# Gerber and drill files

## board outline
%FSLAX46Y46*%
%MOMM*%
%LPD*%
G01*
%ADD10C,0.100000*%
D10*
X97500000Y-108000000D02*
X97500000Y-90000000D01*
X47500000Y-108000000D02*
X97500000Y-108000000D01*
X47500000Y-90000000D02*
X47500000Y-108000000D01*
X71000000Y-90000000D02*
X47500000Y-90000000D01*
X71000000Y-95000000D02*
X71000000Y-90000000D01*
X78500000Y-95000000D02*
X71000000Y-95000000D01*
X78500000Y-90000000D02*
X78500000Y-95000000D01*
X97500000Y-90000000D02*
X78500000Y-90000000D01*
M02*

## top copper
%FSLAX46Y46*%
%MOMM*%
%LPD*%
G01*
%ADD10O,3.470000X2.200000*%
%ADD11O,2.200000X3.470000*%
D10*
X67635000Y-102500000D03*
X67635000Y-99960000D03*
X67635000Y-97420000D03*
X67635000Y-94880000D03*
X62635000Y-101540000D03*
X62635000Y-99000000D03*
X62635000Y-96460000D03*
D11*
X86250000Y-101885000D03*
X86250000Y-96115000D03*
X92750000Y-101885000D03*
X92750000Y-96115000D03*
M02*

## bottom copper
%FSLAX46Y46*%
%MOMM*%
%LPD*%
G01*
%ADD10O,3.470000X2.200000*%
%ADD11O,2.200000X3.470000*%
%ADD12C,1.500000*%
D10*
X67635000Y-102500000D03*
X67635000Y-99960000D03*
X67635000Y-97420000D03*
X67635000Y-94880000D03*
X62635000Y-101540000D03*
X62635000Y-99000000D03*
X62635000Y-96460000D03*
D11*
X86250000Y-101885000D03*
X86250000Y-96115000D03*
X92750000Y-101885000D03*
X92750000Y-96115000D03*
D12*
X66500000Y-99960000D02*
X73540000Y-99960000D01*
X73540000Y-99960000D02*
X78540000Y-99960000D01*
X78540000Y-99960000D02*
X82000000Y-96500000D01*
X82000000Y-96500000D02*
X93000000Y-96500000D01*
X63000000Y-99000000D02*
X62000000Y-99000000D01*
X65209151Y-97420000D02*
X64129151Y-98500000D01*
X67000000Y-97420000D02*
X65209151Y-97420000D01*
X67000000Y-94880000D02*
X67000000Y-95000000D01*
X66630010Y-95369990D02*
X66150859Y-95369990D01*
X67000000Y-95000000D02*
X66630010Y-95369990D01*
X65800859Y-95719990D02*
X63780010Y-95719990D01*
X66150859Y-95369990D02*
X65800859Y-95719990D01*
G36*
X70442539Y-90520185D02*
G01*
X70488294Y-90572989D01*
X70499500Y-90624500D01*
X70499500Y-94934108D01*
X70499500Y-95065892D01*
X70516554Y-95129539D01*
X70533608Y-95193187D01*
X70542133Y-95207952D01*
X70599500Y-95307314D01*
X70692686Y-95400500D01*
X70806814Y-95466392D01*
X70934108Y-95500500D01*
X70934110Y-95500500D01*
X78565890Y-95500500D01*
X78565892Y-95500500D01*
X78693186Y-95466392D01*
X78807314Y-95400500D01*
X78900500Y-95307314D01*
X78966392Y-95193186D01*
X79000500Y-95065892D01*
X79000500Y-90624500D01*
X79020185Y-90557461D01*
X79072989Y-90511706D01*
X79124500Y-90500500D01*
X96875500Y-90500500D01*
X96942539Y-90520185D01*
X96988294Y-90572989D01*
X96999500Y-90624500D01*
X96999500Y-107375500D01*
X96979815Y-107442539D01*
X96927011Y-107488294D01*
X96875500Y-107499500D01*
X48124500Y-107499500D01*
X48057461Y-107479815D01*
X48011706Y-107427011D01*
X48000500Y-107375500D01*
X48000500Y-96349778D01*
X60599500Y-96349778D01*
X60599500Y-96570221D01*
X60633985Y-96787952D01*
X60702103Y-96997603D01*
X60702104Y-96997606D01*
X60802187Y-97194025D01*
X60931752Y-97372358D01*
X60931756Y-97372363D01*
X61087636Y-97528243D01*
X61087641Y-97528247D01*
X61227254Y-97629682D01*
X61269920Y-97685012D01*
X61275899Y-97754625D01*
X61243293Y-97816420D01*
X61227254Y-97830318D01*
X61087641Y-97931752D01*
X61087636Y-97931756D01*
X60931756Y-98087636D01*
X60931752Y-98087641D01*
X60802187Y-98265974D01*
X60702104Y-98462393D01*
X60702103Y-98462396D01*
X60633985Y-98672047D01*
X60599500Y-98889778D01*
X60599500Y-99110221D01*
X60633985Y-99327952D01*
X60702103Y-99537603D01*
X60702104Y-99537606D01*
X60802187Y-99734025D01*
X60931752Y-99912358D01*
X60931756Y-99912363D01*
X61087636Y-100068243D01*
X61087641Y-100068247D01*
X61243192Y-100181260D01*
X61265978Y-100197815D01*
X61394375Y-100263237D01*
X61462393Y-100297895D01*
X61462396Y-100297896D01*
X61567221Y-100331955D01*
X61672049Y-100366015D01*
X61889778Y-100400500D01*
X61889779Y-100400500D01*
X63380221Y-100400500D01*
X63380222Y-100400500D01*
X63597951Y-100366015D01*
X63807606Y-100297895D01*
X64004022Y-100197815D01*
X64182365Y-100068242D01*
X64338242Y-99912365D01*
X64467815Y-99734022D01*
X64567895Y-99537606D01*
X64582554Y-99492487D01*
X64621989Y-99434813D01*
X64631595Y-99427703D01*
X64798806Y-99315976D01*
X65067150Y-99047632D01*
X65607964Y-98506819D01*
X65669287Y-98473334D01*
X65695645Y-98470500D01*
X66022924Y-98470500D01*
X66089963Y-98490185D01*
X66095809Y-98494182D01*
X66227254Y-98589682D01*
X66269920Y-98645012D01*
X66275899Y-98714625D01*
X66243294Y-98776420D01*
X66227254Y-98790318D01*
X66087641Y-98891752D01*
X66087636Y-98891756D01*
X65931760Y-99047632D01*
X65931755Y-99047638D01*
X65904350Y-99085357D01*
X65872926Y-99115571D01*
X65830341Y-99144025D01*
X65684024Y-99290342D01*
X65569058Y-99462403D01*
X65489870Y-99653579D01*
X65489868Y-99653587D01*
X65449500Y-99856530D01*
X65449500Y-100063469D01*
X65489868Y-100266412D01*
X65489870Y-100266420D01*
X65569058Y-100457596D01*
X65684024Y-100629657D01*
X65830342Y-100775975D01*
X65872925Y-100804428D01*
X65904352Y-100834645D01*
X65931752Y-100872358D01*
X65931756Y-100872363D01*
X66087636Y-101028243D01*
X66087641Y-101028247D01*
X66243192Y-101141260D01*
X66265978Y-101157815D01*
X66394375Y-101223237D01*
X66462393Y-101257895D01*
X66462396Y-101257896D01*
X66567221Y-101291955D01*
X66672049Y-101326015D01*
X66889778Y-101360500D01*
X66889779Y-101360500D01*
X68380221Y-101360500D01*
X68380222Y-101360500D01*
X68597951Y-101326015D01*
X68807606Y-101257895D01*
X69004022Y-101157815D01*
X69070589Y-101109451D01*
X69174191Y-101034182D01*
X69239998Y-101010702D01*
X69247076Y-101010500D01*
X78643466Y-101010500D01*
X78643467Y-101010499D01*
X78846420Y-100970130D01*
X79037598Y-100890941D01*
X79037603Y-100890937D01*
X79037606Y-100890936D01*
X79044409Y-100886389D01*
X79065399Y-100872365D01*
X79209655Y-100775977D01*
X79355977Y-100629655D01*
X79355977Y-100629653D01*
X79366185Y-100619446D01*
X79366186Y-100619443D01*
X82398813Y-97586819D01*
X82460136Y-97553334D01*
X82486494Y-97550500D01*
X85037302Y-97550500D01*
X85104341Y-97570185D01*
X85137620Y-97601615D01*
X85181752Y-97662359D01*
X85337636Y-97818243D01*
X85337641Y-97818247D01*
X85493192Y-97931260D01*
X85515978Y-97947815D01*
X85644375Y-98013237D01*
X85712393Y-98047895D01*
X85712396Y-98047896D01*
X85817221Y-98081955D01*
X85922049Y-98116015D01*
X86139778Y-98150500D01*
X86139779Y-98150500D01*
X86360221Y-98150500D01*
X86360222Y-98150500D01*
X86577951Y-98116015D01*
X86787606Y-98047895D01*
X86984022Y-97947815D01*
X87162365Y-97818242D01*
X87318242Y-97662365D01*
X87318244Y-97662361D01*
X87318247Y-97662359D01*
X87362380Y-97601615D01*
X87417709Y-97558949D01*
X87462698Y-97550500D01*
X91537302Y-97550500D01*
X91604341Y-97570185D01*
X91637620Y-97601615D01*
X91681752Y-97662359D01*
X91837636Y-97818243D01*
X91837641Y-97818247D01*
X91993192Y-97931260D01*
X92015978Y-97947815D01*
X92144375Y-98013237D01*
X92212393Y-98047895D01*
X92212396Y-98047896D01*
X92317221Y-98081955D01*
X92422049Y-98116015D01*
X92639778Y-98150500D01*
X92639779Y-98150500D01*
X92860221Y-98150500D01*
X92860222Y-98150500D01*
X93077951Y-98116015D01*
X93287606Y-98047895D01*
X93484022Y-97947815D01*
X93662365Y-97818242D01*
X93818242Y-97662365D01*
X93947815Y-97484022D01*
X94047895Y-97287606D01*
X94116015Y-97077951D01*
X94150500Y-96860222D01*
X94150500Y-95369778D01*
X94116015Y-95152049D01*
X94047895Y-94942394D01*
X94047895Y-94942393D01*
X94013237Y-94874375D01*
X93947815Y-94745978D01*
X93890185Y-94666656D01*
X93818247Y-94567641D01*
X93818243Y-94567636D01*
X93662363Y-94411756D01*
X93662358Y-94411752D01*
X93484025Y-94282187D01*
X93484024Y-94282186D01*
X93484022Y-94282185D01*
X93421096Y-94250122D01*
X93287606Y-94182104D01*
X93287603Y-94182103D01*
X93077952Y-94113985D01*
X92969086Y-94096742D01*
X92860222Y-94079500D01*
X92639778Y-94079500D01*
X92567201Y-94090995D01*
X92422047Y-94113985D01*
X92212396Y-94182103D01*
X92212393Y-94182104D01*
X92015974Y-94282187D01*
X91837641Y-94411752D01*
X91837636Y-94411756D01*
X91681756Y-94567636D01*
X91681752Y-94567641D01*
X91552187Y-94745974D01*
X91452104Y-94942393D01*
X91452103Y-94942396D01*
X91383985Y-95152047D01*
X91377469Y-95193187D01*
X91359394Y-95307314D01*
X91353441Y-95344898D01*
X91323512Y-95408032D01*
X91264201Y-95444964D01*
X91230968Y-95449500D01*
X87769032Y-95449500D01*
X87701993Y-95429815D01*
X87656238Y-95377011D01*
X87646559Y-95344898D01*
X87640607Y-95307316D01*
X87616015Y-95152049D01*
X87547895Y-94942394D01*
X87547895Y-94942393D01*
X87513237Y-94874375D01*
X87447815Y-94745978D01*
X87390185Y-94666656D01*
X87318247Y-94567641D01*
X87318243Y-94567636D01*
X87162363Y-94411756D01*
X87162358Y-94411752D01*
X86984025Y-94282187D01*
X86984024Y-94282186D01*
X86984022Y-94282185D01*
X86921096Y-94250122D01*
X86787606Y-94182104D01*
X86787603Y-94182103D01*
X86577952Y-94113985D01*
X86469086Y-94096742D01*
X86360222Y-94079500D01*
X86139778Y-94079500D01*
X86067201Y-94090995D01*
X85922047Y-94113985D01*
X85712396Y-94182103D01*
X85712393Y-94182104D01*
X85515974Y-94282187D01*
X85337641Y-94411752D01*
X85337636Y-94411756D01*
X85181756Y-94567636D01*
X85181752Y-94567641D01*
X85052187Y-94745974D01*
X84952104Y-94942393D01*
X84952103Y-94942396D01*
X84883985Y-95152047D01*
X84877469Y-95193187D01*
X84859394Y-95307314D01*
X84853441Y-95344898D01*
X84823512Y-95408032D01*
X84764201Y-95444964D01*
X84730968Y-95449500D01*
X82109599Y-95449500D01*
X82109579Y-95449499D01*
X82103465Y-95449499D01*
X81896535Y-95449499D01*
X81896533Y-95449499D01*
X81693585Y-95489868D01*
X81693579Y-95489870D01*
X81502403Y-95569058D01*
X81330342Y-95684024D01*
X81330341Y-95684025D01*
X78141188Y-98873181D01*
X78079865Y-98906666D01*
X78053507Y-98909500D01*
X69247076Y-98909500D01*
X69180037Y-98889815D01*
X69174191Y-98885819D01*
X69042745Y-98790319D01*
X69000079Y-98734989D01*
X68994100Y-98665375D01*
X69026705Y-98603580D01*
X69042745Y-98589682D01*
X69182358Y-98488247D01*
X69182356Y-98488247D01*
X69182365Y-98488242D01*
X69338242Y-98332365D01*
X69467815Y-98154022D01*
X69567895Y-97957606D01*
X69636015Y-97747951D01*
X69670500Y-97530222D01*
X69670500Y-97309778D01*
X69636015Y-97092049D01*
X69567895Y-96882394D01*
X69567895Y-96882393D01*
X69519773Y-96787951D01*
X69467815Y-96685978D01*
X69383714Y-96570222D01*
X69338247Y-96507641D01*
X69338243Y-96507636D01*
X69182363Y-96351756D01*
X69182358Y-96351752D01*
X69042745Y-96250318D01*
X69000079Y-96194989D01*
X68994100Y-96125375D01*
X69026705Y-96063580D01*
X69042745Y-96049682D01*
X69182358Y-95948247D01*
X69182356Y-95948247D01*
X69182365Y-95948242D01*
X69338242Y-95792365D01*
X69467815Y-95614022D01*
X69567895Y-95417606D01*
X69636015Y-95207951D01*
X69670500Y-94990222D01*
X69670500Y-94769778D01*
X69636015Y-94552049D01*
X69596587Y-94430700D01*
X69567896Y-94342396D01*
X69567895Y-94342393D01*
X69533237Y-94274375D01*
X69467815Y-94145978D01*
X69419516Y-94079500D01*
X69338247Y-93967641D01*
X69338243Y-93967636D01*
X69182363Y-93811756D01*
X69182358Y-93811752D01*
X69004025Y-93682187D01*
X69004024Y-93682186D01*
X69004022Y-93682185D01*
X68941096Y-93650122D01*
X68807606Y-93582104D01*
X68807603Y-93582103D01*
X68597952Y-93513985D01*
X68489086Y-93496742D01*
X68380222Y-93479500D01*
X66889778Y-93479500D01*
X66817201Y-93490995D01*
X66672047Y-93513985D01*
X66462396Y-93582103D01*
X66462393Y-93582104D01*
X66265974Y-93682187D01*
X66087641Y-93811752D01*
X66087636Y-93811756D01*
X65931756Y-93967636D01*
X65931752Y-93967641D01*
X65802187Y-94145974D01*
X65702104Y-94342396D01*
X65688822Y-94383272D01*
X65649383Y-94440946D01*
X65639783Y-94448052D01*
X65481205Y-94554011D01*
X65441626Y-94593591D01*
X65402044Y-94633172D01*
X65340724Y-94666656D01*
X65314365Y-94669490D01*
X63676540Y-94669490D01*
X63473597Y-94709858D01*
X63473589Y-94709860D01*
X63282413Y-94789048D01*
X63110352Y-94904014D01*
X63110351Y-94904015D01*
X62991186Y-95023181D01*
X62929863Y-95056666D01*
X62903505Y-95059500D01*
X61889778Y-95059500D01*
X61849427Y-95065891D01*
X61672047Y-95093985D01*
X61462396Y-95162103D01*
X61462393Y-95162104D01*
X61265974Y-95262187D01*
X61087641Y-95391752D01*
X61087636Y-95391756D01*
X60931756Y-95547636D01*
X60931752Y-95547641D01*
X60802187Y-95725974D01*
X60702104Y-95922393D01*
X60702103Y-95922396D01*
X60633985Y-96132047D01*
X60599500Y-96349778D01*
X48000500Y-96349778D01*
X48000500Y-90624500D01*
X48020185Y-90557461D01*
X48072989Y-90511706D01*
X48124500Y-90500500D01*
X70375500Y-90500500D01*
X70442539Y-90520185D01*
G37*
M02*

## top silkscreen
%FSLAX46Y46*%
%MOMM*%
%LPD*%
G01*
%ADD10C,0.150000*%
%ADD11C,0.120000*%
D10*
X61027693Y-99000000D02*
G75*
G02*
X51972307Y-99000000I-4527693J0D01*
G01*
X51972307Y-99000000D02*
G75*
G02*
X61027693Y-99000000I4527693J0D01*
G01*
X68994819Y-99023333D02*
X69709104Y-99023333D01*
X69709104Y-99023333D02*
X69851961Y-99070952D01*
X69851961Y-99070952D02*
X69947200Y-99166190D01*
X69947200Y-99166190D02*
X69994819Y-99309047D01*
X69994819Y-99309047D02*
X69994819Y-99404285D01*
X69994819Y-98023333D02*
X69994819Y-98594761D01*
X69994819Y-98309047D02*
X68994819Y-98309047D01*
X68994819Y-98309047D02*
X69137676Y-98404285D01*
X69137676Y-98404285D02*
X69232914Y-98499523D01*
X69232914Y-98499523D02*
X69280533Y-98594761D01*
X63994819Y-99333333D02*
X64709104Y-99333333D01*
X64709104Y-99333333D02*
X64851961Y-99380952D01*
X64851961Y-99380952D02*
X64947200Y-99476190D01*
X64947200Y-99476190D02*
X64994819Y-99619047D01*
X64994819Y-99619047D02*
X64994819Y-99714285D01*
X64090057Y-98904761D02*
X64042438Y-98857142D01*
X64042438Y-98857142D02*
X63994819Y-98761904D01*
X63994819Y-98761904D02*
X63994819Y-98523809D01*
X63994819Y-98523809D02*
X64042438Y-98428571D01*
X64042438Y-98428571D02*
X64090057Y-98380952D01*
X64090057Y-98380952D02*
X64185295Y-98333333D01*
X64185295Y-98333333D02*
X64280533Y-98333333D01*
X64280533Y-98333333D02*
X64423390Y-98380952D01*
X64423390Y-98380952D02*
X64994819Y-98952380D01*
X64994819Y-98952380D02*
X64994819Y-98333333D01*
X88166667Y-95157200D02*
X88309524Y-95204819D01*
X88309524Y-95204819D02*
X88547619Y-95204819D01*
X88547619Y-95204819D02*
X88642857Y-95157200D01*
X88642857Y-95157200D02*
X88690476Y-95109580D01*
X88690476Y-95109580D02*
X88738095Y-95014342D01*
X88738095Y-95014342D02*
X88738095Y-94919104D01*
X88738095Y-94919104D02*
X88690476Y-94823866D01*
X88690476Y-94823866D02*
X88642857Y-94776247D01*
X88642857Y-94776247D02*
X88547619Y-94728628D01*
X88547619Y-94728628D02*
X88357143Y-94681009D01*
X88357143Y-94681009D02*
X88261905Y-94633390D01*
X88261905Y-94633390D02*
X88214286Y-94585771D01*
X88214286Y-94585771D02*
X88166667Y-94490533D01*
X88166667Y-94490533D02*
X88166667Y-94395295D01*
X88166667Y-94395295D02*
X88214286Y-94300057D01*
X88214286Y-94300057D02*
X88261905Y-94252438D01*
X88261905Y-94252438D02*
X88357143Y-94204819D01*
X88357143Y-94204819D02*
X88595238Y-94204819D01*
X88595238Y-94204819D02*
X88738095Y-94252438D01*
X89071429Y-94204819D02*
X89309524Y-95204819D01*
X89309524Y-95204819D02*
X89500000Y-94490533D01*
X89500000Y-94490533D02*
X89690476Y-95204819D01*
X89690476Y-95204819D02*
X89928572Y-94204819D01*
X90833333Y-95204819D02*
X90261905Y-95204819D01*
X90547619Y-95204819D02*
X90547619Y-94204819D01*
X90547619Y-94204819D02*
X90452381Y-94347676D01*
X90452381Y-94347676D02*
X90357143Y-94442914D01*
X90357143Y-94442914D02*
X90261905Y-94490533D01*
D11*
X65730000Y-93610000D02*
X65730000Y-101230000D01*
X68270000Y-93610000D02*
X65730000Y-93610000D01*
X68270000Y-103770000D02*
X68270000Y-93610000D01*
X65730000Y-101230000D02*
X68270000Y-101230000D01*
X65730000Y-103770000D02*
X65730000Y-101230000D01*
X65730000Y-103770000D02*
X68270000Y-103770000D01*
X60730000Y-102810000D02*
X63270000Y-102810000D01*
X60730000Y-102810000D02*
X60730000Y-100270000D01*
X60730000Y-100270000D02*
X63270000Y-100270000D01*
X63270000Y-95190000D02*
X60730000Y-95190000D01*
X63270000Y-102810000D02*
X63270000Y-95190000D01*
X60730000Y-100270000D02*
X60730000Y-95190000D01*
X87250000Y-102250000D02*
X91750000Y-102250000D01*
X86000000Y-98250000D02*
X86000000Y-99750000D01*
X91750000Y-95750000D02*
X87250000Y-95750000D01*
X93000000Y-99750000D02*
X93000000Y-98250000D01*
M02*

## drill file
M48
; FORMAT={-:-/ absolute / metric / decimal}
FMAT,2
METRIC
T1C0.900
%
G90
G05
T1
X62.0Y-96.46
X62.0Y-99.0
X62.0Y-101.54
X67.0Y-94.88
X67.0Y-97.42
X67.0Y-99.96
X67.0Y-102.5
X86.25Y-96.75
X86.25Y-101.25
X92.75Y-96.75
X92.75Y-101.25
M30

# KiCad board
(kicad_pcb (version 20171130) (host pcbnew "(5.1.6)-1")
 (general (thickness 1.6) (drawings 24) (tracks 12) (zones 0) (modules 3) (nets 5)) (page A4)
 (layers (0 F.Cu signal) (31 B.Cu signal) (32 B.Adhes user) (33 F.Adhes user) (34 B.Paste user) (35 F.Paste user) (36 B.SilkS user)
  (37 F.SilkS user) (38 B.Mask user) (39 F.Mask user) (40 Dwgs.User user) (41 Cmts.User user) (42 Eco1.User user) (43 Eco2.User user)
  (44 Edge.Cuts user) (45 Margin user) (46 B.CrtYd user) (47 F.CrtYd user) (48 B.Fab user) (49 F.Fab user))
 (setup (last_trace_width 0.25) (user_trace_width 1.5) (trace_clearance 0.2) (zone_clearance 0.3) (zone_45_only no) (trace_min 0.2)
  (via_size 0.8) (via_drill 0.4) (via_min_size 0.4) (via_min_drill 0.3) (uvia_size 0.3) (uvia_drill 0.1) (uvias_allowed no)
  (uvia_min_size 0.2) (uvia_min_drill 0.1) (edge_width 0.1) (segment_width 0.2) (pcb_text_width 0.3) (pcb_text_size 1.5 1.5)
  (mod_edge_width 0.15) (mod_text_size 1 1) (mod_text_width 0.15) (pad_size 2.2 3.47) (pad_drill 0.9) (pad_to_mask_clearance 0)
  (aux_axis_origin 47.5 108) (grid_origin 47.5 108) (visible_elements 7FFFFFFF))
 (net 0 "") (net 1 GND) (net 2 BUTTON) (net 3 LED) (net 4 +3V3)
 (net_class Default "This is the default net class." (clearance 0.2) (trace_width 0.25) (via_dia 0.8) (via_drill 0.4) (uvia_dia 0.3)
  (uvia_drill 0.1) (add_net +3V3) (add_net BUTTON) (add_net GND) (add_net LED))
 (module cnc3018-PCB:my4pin (layer F.Cu) (at 67 102.5 90)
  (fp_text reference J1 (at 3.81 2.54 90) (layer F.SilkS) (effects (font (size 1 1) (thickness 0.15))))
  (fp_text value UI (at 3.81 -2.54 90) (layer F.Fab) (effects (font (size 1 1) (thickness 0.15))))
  (fp_line (start 8.89 -1.27) (end 1.27 -1.27) (layer F.SilkS) (width 0.12))
  (fp_line (start 8.89 1.27) (end 8.89 -1.27) (layer F.SilkS) (width 0.12))
  (fp_line (start -1.27 1.27) (end 8.89 1.27) (layer F.SilkS) (width 0.12))
  (fp_line (start 1.27 -1.27) (end 1.27 1.27) (layer F.SilkS) (width 0.12))
  (fp_line (start -1.27 -1.27) (end 1.27 -1.27) (layer F.SilkS) (width 0.12))
  (fp_line (start -1.27 -1.27) (end -1.27 1.27) (layer F.SilkS) (width 0.12))
  (pad 1 thru_hole oval (at 0 0 90) (size 2.2 3.47) (drill 0.9 (offset 0 0.635)) (layers *.Cu *.Mask) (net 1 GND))
  (pad 2 thru_hole oval (at 2.54 0 90) (size 2.2 3.47) (drill 0.9 (offset 0 0.635)) (layers *.Cu *.Mask) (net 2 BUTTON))
  (pad 3 thru_hole oval (at 5.08 0 90) (size 2.2 3.47) (drill 0.9 (offset 0 0.635)) (layers *.Cu *.Mask) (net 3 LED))
  (pad 4 thru_hole oval (at 7.62 0 90) (size 2.2 3.47) (drill 0.9 (offset 0 0.635)) (layers *.Cu *.Mask) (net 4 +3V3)))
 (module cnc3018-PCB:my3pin (layer F.Cu) (at 62 99 90)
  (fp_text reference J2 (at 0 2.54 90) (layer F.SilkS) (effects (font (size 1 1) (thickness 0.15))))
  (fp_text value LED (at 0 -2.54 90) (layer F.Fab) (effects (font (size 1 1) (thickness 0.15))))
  (fp_line (start -3.81 -1.27) (end -3.81 1.27) (layer F.SilkS) (width 0.12))
  (fp_line (start -3.81 -1.27) (end -1.27 -1.27) (layer F.SilkS) (width 0.12))
  (fp_line (start -1.27 -1.27) (end -1.27 1.27) (layer F.SilkS) (width 0.12))
  (fp_line (start 3.81 1.27) (end 3.81 -1.27) (layer F.SilkS) (width 0.12))
  (fp_line (start -3.81 1.27) (end 3.81 1.27) (layer F.SilkS) (width 0.12))
  (fp_line (start -1.27 -1.27) (end 3.81 -1.27) (layer F.SilkS) (width 0.12))
  (pad 1 thru_hole oval (at -2.54 0 90) (size 2.2 3.47) (drill 0.9 (offset 0 0.635)) (layers *.Cu *.Mask) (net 1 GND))
  (pad 2 thru_hole oval (at 0 0 90) (size 2.2 3.47) (drill 0.9 (offset 0 0.635)) (layers *.Cu *.Mask) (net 3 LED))
  (pad 3 thru_hole oval (at 2.54 0 90) (size 2.2 3.47) (drill 0.9 (offset 0 0.635)) (layers *.Cu *.Mask) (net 4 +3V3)))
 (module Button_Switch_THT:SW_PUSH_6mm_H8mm (layer F.Cu) (at 86.25 96.75)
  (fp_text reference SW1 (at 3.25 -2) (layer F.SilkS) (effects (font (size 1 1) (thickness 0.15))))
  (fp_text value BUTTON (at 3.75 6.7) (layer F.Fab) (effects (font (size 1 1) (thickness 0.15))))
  (fp_line (start 1 5.5) (end 5.5 5.5) (layer F.SilkS) (width 0.12))
  (fp_line (start -0.25 1.5) (end -0.25 3) (layer F.SilkS) (width 0.12))
  (fp_line (start 5.5 -1) (end 1 -1) (layer F.SilkS) (width 0.12))
  (fp_line (start 6.75 3) (end 6.75 1.5) (layer F.SilkS) (width 0.12))
  (pad 2 thru_hole oval (at 0 4.5) (size 2.2 3.47) (drill 0.9 (offset 0 0.635)) (layers *.Cu *.Mask) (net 1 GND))
  (pad 1 thru_hole oval (at 0 0) (size 2.2 3.47) (drill 0.9 (offset 0 -0.635)) (layers *.Cu *.Mask) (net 2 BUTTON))
  (pad 2 thru_hole oval (at 6.5 4.5) (size 2.2 3.47) (drill 0.9 (offset 0 0.635)) (layers *.Cu *.Mask) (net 1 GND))
  (pad 1 thru_hole oval (at 6.5 0) (size 2.2 3.47) (drill 0.9 (offset 0 -0.635)) (layers *.Cu *.Mask) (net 2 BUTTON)))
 (gr_line (start 97.5 108) (end 97.5 90) (layer Edge.Cuts) (width 0.1))
 (gr_line (start 47.5 108) (end 97.5 108) (layer Edge.Cuts) (width 0.1))
 (gr_line (start 47.5 90) (end 47.5 108) (layer Edge.Cuts) (width 0.1))
 (gr_line (start 71 90) (end 47.5 90) (layer Edge.Cuts) (width 0.1))
 (gr_line (start 71 95) (end 71 90) (layer Edge.Cuts) (width 0.1))
 (gr_line (start 78.5 95) (end 71 95) (layer Edge.Cuts) (width 0.1))
 (gr_line (start 78.5 90) (end 78.5 95) (layer Edge.Cuts) (width 0.1))
 (gr_line (start 97.5 90) (end 78.5 90) (layer Edge.Cuts) (width 0.1))
 (gr_circle (center 56.5 99) (end 61.027693 99) (layer F.SilkS) (width 0.15))
 (segment (start 66.5 99.96) (end 73.54 99.96) (width 1.5) (layer B.Cu) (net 2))
 (segment (start 73.54 99.96) (end 78.54 99.96) (width 1.5) (layer B.Cu) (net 2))
 (segment (start 78.54 99.96) (end 82 96.5) (width 1.5) (layer B.Cu) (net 2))
 (segment (start 82 96.5) (end 93 96.5) (width 1.5) (layer B.Cu) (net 2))
 (segment (start 63 99) (end 62 99) (width 1.5) (layer B.Cu) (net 3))
 (segment (start 65.209151 97.42) (end 64.129151 98.5) (width 1.5) (layer B.Cu) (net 3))
 (segment (start 67 97.42) (end 65.209151 97.42) (width 1.5) (layer B.Cu) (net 3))
 (segment (start 67 94.88) (end 67 95) (width 1.5) (layer B.Cu) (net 4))
 (segment (start 66.63001 95.36999) (end 66.150859 95.36999) (width 1.5) (layer B.Cu) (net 4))
 (segment (start 67 95) (end 66.63001 95.36999) (width 1.5) (layer B.Cu) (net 4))
 (segment (start 65.800859 95.71999) (end 63.78001 95.71999) (width 1.5) (layer B.Cu) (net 4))
 (segment (start 66.150859 95.36999) (end 65.800859 95.71999) (width 1.5) (layer B.Cu) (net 4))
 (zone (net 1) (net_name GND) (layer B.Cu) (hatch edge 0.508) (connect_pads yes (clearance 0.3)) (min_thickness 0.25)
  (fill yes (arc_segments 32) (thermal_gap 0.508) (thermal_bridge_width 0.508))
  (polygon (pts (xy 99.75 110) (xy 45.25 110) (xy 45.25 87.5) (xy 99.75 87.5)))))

